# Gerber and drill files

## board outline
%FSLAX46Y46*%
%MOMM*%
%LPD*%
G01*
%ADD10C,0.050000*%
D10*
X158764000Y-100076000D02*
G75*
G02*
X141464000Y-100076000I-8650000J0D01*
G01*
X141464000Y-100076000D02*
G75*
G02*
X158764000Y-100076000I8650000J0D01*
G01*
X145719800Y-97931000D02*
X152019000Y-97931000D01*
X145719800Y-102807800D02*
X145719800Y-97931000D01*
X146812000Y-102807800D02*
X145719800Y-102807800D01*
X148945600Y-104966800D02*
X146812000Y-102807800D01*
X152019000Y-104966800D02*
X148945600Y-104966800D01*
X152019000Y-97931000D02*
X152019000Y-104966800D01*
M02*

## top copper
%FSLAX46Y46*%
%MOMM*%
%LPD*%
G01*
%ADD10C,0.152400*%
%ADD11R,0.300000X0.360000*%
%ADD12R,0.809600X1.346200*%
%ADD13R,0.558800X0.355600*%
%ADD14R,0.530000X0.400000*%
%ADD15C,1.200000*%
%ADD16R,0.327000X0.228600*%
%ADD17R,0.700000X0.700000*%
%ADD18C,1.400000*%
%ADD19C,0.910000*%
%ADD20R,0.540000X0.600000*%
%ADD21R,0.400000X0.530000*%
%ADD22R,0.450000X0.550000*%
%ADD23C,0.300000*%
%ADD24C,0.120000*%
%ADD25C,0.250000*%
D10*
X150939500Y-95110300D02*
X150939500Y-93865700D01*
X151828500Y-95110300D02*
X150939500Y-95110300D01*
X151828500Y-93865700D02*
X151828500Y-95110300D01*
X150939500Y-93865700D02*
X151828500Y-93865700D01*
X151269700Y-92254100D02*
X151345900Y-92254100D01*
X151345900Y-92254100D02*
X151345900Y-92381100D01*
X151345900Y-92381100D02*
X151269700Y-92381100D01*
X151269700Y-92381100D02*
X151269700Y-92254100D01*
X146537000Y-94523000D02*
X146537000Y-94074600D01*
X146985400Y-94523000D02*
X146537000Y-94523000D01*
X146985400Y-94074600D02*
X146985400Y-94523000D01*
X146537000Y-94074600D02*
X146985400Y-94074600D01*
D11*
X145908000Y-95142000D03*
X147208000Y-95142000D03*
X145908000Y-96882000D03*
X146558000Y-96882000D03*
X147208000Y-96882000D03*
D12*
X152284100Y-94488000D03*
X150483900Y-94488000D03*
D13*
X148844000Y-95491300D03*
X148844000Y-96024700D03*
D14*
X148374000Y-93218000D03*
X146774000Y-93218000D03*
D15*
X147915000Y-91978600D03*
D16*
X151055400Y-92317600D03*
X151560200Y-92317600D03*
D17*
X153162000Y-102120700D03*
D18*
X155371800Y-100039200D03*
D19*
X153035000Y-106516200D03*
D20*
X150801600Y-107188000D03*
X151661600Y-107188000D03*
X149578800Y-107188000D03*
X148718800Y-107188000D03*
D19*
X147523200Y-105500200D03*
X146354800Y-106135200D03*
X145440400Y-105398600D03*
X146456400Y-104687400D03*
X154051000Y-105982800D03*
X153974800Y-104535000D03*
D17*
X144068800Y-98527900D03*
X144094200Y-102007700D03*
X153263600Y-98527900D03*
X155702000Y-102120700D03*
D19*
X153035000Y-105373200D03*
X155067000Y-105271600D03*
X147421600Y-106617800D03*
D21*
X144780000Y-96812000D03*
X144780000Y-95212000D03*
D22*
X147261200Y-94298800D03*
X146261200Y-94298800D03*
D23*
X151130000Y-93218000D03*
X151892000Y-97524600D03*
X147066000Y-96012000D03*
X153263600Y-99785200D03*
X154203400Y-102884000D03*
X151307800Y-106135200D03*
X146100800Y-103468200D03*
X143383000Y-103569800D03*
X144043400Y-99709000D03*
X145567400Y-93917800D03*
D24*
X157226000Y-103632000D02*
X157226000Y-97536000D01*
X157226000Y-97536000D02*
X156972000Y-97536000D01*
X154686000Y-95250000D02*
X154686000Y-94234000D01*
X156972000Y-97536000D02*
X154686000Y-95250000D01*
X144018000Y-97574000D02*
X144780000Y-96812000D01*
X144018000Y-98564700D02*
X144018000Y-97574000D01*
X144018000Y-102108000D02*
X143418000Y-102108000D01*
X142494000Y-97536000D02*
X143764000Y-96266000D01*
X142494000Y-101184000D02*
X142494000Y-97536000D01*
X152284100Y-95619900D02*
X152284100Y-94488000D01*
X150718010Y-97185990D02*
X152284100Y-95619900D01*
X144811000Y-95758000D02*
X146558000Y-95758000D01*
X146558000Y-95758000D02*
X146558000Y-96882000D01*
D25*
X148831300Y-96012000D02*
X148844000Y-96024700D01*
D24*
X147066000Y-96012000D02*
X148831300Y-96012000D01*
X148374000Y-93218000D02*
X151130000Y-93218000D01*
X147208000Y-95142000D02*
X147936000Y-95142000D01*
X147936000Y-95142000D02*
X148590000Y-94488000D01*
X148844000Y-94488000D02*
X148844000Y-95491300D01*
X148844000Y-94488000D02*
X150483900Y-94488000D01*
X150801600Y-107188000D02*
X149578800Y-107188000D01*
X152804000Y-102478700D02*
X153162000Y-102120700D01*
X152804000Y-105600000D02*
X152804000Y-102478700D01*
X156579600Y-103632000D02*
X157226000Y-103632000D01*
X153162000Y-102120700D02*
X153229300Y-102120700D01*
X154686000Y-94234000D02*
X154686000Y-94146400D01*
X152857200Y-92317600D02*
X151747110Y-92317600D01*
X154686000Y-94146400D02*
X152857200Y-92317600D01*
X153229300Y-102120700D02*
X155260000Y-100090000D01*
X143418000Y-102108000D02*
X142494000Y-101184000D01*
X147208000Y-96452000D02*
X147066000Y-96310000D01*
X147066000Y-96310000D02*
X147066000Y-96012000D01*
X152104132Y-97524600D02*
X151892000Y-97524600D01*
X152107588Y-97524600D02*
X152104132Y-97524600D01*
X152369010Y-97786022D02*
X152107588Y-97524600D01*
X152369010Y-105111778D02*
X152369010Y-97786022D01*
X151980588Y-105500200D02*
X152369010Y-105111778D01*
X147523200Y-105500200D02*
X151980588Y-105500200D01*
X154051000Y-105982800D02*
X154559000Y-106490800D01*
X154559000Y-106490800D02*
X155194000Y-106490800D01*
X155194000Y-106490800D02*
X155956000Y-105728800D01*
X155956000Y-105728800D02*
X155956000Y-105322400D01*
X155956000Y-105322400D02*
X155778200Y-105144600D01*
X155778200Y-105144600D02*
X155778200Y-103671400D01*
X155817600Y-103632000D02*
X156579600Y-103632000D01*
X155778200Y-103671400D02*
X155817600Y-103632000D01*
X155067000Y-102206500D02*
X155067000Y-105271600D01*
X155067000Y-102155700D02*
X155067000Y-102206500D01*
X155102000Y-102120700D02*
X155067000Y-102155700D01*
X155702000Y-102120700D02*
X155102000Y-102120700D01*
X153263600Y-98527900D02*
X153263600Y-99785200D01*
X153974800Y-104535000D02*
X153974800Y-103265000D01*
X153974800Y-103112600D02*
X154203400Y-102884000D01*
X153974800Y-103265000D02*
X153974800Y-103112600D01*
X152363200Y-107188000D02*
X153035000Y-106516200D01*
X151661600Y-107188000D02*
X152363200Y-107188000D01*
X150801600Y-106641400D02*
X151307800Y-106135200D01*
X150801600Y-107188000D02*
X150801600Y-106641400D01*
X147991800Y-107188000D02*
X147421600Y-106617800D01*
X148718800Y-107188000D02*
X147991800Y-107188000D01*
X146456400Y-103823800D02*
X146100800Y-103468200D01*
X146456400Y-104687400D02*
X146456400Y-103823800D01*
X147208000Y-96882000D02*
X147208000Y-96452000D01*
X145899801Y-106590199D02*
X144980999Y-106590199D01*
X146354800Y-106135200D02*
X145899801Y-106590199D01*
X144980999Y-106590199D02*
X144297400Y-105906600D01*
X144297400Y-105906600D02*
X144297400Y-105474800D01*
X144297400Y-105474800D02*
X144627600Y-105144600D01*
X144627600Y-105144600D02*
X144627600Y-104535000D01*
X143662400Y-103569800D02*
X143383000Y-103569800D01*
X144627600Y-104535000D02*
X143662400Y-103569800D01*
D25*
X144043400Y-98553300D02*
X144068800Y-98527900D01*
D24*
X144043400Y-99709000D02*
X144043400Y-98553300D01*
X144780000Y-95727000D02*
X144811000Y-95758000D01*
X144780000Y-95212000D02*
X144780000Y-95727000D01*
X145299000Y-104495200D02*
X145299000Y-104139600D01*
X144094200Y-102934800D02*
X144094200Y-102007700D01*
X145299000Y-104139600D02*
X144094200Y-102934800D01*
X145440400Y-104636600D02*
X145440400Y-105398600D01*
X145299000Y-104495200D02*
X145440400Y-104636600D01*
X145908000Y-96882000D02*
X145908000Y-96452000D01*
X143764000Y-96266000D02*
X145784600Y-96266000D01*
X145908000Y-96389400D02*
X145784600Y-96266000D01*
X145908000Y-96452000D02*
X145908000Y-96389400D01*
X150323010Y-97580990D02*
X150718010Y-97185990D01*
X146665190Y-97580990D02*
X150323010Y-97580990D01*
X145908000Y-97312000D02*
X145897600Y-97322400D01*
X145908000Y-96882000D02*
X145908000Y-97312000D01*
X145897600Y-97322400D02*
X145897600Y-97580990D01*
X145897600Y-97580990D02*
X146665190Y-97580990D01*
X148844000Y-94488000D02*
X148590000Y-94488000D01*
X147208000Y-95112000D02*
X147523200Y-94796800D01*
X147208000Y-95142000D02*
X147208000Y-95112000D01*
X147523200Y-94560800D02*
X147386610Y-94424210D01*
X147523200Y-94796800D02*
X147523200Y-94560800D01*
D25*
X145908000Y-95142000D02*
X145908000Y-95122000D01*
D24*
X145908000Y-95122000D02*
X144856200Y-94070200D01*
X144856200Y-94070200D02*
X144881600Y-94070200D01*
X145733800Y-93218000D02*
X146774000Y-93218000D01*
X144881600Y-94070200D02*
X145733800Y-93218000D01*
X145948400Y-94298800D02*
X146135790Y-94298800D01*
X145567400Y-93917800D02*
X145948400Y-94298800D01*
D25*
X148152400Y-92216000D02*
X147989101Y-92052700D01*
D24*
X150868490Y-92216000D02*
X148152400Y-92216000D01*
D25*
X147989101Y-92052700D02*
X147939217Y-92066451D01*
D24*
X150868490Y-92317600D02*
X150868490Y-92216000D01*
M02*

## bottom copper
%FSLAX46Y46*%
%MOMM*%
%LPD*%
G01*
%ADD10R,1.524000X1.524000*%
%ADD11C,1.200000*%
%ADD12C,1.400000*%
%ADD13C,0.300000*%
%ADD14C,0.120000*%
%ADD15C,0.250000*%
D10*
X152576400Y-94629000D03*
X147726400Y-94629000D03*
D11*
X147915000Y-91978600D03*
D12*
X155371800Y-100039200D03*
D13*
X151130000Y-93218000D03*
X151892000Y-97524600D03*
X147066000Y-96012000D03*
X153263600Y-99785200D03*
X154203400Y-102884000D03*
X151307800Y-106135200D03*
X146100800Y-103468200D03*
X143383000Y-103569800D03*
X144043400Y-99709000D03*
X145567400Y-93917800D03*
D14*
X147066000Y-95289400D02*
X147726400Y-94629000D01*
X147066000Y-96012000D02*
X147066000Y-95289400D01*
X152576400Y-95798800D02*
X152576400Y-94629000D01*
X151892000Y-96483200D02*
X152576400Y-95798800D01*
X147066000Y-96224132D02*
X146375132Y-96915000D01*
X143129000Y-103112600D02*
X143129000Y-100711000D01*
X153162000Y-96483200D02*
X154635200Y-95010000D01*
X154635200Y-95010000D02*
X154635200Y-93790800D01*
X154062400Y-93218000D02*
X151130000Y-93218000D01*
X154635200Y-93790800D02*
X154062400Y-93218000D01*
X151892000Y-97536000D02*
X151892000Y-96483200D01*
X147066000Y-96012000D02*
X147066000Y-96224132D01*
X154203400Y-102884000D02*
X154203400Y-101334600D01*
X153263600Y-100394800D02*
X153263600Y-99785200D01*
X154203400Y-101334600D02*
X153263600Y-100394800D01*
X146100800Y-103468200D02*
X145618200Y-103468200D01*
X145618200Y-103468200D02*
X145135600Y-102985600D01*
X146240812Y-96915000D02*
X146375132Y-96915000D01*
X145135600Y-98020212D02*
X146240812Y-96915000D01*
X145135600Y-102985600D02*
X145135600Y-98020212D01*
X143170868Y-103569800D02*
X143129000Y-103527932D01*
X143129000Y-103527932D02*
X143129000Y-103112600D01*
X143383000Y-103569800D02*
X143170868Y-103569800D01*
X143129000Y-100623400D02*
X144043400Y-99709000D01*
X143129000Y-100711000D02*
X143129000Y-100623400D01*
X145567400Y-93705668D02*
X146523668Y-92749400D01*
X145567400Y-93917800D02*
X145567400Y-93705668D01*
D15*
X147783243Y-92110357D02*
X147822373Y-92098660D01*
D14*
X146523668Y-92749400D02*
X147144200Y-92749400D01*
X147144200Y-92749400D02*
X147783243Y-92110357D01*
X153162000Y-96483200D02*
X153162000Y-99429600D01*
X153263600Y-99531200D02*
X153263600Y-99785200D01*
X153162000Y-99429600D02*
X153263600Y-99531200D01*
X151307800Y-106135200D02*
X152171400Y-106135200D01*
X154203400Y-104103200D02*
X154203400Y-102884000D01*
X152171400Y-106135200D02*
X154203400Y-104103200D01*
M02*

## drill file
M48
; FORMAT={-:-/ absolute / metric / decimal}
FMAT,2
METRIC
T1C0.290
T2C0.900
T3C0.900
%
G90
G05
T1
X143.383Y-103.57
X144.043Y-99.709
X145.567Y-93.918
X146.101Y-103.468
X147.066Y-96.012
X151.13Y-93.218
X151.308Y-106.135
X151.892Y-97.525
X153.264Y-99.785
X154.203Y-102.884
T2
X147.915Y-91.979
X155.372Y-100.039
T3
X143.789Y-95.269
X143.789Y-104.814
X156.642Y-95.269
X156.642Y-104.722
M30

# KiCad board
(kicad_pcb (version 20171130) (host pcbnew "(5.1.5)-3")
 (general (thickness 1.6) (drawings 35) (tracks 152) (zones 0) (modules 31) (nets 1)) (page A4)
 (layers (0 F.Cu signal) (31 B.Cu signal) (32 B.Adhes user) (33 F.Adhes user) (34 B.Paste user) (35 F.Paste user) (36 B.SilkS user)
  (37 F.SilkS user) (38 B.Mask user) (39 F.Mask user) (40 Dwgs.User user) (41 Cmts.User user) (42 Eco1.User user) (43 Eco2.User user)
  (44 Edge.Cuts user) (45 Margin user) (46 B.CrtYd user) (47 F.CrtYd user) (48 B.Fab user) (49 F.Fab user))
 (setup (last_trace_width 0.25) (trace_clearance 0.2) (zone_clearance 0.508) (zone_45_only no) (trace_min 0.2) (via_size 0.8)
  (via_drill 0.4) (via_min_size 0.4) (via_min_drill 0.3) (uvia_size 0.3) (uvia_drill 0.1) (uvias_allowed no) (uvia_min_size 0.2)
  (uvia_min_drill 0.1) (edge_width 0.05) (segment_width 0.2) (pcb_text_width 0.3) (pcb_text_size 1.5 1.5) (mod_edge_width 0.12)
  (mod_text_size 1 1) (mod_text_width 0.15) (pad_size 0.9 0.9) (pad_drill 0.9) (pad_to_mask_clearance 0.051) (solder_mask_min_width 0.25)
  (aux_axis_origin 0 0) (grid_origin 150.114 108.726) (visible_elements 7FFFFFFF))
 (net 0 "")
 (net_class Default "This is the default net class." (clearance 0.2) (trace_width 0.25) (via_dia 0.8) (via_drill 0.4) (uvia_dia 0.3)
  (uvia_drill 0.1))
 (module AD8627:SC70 (layer F.Cu) (at 146.558 96.012)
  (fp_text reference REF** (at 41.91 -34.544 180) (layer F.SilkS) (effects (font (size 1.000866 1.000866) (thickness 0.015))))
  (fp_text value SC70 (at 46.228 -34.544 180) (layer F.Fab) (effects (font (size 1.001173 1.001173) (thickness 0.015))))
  (pad 5 smd rect (at -0.65 -0.87 180) (size 0.3 0.36) (layers F.Cu F.Paste F.Mask))
  (pad 4 smd rect (at 0.65 -0.87 180) (size 0.3 0.36) (layers F.Cu F.Paste F.Mask))
  (pad 1 smd rect (at -0.65 0.87) (size 0.3 0.36) (layers F.Cu F.Paste F.Mask))
  (pad 2 smd rect (at 0 0.87) (size 0.3 0.36) (layers F.Cu F.Paste F.Mask))
  (pad 3 smd rect (at 0.65 0.87) (size 0.3 0.36) (layers F.Cu F.Paste F.Mask)))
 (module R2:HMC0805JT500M (layer F.Cu) (at 151.384 94.488)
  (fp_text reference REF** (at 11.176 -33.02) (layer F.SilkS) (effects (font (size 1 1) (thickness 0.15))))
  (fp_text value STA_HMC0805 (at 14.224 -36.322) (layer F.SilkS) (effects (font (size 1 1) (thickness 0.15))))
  (fp_line (start -0.4445 0.6223) (end -0.4445 -0.6223) (layer F.Cu) (width 0.1524))
  (fp_line (start 0.4445 0.6223) (end -0.4445 0.6223) (layer F.Cu) (width 0.1524))
  (fp_line (start 0.4445 -0.6223) (end 0.4445 0.6223) (layer F.Cu) (width 0.1524))
  (fp_line (start -0.4445 -0.6223) (end 0.4445 -0.6223) (layer F.Cu) (width 0.1524))
  (pad 2 smd rect (at 0.9001 0) (size 0.8096 1.3462) (layers F.Cu F.Paste F.Mask))
  (pad 1 smd rect (at -0.9001 0) (size 0.8096 1.3462) (layers F.Cu F.Paste F.Mask)))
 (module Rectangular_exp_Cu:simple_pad (layer F.Cu) (at 150.2664 94.629)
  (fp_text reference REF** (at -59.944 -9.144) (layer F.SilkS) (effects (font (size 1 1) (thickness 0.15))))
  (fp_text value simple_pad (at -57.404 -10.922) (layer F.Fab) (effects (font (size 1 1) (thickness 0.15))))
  (pad 2 smd rect (at 2.31 0) (size 1.524 1.524) (layers B.Cu))
  (pad 1 smd rect (at -2.54 0) (size 1.524 1.524) (layers B.Cu)))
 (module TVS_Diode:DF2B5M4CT (layer F.Cu) (at 148.844 95.758 90)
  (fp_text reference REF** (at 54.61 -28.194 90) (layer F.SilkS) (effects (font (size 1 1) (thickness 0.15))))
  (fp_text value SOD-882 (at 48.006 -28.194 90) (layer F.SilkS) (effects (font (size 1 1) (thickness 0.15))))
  (pad 2 smd rect (at 0.2667 0 90) (size 0.3556 0.5588) (layers F.Cu F.Paste F.Mask))
  (pad 1 smd rect (at -0.2667 0 90) (size 0.3556 0.5588) (layers F.Cu F.Paste F.Mask)))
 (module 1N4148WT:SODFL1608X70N (layer F.Cu) (at 147.574 93.218)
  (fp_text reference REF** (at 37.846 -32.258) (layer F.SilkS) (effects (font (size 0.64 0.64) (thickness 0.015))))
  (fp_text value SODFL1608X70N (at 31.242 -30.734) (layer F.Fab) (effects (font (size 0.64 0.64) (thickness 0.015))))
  (pad A smd rect (at 0.8 0) (size 0.53 0.4) (layers F.Cu F.Paste F.Mask))
  (pad C smd rect (at -0.8 0) (size 0.53 0.4) (layers F.Cu F.Paste F.Mask)))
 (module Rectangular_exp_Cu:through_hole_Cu (layer F.Cu) (at 148.209 92.47)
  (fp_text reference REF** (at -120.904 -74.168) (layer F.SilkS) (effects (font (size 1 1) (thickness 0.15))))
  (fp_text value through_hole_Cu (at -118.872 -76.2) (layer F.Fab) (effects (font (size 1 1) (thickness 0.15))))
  (pad 1 thru_hole circle (at -0.294 -0.4914) (size 1.2 1.2) (drill 0.9) (layers *.Mask F.Cu)))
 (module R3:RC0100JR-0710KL (layer F.Cu) (at 151.3078 92.3176)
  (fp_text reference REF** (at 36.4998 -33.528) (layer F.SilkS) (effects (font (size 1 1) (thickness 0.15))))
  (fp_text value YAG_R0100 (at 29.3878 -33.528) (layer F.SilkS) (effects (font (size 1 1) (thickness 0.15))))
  (fp_line (start -0.0381 -0.0635) (end 0.0381 -0.0635) (layer F.Cu) (width 0.1524))
  (fp_line (start 0.0381 -0.0635) (end 0.0381 0.0635) (layer F.Cu) (width 0.1524))
  (fp_line (start 0.0381 0.0635) (end -0.0381 0.0635) (layer F.Cu) (width 0.1524))
  (fp_line (start -0.0381 0.0635) (end -0.0381 -0.0635) (layer F.Cu) (width 0.1524))
  (pad 1 smd rect (at -0.2524 0) (size 0.327 0.2286) (layers F.Cu F.Paste F.Mask))
  (pad 2 smd rect (at 0.2524 0) (size 0.327 0.2286) (layers F.Cu F.Paste F.Mask)))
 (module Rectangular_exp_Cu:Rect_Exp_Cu (layer F.Cu) (at 153.162 102.108)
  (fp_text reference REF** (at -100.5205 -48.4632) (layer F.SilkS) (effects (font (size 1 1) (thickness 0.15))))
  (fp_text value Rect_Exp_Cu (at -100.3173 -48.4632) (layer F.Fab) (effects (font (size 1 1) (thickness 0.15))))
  (pad 1 smd rect (at 0 0.0127) (size 0.7 0.7) (layers F.Cu F.Paste F.Mask)))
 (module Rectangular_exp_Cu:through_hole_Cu (layer F.Cu) (at 156.0678 99.0092)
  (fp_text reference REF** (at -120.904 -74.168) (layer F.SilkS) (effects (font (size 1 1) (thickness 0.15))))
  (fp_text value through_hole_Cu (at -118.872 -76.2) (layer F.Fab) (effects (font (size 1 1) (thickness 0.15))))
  (pad 1 thru_hole circle (at -0.696 1.03) (size 1.4 1.4) (drill 0.9) (layers *.Mask F.Cu)))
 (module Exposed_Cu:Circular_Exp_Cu (layer F.Cu) (at 152.885 106.7302)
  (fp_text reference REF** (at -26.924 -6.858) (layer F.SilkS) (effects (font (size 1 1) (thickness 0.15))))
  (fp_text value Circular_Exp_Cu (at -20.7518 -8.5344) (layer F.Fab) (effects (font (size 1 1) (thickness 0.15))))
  (pad 1 smd circle (at 0.15 -0.214) (size 0.91 0.91) (layers F.Cu F.Paste F.Mask)))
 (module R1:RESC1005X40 (layer F.Cu) (at 151.2316 107.188)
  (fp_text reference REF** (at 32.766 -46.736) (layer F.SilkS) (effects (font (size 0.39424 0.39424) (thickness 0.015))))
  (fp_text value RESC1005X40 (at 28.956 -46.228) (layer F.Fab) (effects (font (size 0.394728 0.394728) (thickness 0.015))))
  (pad 1 smd rect (at -0.43 0) (size 0.54 0.6) (layers F.Cu F.Paste F.Mask))
  (pad 2 smd rect (at 0.43 0) (size 0.54 0.6) (layers F.Cu F.Paste F.Mask)))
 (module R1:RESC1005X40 (layer F.Cu) (at 149.1488 107.188)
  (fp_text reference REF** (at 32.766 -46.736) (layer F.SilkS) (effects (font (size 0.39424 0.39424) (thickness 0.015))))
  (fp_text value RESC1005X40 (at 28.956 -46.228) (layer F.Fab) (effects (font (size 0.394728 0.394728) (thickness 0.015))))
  (pad 2 smd rect (at 0.43 0) (size 0.54 0.6) (layers F.Cu F.Paste F.Mask))
  (pad 1 smd rect (at -0.43 0) (size 0.54 0.6) (layers F.Cu F.Paste F.Mask)))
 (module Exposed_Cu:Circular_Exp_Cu (layer F.Cu) (at 147.8032 105.8182)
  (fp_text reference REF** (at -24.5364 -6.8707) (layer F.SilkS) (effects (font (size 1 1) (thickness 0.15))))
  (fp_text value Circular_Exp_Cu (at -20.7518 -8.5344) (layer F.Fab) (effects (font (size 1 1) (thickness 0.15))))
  (pad 1 smd circle (at -0.28 -0.318) (size 0.91 0.91) (layers F.Cu F.Paste F.Mask)))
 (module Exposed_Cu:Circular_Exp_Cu (layer F.Cu) (at 146.7268 106.3562)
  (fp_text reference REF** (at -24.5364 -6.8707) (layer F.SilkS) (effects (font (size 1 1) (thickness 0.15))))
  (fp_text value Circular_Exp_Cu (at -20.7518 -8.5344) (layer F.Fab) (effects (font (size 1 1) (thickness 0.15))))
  (pad 1 smd circle (at -0.372 -0.221) (size 0.91 0.91) (layers F.Cu F.Paste F.Mask)))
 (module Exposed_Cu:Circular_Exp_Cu (layer F.Cu) (at 145.3786 105.5118)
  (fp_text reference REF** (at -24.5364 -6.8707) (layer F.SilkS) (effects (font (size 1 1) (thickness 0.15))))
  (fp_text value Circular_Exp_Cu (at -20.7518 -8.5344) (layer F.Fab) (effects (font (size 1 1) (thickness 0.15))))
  (pad 1 smd circle (at 0.0618 -0.1132) (size 0.91 0.91) (layers F.Cu F.Paste F.Mask)))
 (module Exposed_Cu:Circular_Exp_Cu (layer F.Cu) (at 146.7554 105.2854)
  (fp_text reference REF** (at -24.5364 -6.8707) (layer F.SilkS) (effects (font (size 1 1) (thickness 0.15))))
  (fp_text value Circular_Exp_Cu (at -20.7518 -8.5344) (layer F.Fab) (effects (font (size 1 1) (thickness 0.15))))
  (pad 1 smd circle (at -0.299 -0.598) (size 0.91 0.91) (layers F.Cu F.Paste F.Mask)))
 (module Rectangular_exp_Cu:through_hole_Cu (layer F.Cu) (at 160.8582 95.518)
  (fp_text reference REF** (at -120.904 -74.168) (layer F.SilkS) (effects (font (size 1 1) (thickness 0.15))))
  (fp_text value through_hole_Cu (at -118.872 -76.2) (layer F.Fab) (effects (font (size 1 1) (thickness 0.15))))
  (pad "" np_thru_hole circle (at -4.2158 -0.249) (size 0.9 0.9) (drill 0.9) (layers *.Cu *.Mask)))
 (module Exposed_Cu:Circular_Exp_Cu (layer F.Cu) (at 153.645 106.4578)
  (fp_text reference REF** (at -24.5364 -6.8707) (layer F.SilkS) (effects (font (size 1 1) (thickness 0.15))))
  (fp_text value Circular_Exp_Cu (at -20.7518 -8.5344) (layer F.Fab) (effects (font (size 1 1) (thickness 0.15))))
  (pad 1 smd circle (at 0.406 -0.475) (size 0.91 0.91) (layers F.Cu F.Paste F.Mask)))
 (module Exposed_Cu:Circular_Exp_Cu (layer F.Cu) (at 153.9228 105.133)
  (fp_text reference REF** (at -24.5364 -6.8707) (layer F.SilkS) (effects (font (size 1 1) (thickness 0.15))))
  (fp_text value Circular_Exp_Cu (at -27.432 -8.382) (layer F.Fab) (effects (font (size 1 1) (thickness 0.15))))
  (pad 1 smd circle (at 0.052 -0.598) (size 0.91 0.91) (layers F.Cu F.Paste F.Mask)))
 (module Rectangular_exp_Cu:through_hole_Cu (layer F.Cu) (at 159.4358 103.3412)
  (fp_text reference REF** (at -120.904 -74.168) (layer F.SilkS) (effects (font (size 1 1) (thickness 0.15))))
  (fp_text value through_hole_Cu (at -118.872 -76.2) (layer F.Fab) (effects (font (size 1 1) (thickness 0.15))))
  (pad "" np_thru_hole circle (at -2.7934 1.3806) (size 0.9 0.9) (drill 0.9) (layers *.Cu *.Mask)))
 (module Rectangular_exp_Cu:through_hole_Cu (layer F.Cu) (at 138.6332 103.6484)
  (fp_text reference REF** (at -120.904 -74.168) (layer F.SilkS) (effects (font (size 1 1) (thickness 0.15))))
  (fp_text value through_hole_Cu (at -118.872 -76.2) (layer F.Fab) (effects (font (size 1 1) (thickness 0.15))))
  (pad "" np_thru_hole circle (at 5.1562 1.166) (size 0.9 0.9) (drill 0.9) (layers *.Cu *.Mask)))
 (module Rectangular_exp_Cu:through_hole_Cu (layer F.Cu) (at 141.5832 93.4162)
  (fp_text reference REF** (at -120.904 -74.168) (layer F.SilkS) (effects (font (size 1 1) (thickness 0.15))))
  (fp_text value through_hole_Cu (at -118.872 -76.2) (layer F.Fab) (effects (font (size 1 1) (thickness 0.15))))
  (pad "" np_thru_hole circle (at 2.2062 1.8528) (size 0.9 0.9) (drill 0.9) (layers *.Cu *.Mask)))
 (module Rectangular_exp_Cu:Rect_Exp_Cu (layer F.Cu) (at 144.0688 98.5152)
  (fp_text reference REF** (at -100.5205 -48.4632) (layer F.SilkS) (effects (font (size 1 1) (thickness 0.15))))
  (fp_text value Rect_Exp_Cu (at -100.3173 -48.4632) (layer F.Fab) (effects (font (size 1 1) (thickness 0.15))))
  (pad 1 smd rect (at 0 0.0127) (size 0.7 0.7) (layers F.Cu F.Paste F.Mask)))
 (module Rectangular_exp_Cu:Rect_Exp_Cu (layer F.Cu) (at 144.0942 101.995)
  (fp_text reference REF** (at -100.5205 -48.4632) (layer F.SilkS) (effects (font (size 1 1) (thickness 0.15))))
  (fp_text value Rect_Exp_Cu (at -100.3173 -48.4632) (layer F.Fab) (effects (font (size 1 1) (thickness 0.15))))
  (pad 1 smd rect (at 0 0.0127) (size 0.7 0.7) (layers F.Cu F.Paste F.Mask)))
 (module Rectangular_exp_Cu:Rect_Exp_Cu (layer F.Cu) (at 153.2636 98.5152)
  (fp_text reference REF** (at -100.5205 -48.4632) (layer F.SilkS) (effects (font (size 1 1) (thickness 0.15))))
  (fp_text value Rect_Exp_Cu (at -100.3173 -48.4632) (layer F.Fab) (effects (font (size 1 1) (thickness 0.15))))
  (pad 1 smd rect (at 0 0.0127) (size 0.7 0.7) (layers F.Cu F.Paste F.Mask)))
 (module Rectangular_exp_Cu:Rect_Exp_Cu (layer F.Cu) (at 155.702 102.108)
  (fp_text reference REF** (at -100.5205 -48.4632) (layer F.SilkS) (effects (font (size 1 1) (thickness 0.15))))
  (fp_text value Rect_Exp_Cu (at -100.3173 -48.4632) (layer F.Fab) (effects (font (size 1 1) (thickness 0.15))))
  (pad 1 smd rect (at 0 0.0127) (size 0.7 0.7) (layers F.Cu F.Paste F.Mask)))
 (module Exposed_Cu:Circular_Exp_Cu (layer F.Cu) (at 153.1263 105.6912)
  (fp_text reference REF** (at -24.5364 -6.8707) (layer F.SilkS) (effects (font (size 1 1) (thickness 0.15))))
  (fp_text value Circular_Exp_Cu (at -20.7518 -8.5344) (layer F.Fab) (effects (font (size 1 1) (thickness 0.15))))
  (pad 1 smd circle (at -0.0913 -0.318) (size 0.91 0.91) (layers F.Cu F.Paste F.Mask)))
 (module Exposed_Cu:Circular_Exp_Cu (layer F.Cu) (at 154.431 105.9296)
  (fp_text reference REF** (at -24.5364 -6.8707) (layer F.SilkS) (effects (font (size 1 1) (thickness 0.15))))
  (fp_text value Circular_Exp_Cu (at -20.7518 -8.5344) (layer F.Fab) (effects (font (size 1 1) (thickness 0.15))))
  (pad 1 smd circle (at 0.636 -0.658) (size 0.91 0.91) (layers F.Cu F.Paste F.Mask)))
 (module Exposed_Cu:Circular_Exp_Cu (layer F.Cu) (at 147.7676 106.8318)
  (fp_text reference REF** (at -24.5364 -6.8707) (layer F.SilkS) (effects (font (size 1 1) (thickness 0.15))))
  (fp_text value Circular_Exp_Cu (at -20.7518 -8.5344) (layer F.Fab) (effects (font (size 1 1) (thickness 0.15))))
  (pad 1 smd circle (at -0.346 -0.214) (size 0.91 0.91) (layers F.Cu F.Paste F.Mask)))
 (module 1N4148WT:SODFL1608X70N (layer F.Cu) (at 144.78 96.012 90)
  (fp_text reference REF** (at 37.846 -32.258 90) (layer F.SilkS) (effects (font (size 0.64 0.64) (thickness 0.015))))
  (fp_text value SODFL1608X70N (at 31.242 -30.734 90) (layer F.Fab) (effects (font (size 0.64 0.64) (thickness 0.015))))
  (pad C smd rect (at -0.8 0 90) (size 0.53 0.4) (layers F.Cu F.Paste F.Mask))
  (pad A smd rect (at 0.8 0 90) (size 0.53 0.4) (layers F.Cu F.Paste F.Mask)))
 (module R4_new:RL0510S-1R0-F (layer F.Cu) (at 146.7612 94.2988)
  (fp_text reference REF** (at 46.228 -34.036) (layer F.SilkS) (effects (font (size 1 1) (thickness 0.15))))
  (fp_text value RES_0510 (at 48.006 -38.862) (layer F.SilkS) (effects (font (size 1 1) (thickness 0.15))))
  (fp_line (start -0.2242 0.2242) (end -0.2242 -0.2242) (layer F.Cu) (width 0.1524))
  (fp_line (start 0.2242 0.2242) (end -0.2242 0.2242) (layer F.Cu) (width 0.1524))
  (fp_line (start 0.2242 -0.2242) (end 0.2242 0.2242) (layer F.Cu) (width 0.1524))
  (fp_line (start -0.2242 -0.2242) (end 0.2242 -0.2242) (layer F.Cu) (width 0.1524))
  (pad 2 smd rect (at 0.5 0) (size 0.45 0.55) (layers F.Cu F.Paste F.Mask))
  (pad 1 smd rect (at -0.5 0) (size 0.45 0.55) (layers F.Cu F.Paste F.Mask)))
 (gr_circle (center 150.114 100.076) (end 158.764 100.076) (layer Edge.Cuts) (width 0.05))
 (gr_line (start 145.7198 97.931) (end 152.019 97.931) (layer Edge.Cuts) (width 0.05))
 (gr_line (start 145.7198 102.8078) (end 145.7198 97.931) (layer Edge.Cuts) (width 0.05))
 (gr_line (start 146.812 102.8078) (end 145.7198 102.8078) (layer Edge.Cuts) (width 0.05))
 (gr_line (start 148.9456 104.9668) (end 146.812 102.8078) (layer Edge.Cuts) (width 0.05))
 (gr_line (start 152.019 104.9668) (end 148.9456 104.9668) (layer Edge.Cuts) (width 0.05))
 (gr_line (start 152.019 97.931) (end 152.019 104.9668) (layer Edge.Cuts) (width 0.05))
 (via (at 151.13 93.218) (size 0.3) (drill 0.29) (layers F.Cu B.Cu) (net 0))
 (via (at 151.892 97.5246) (size 0.3) (drill 0.29) (layers F.Cu B.Cu) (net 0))
 (segment (start 157.226 103.632) (end 157.226 97.536) (width 0.12) (layer F.Cu) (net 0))
 (segment (start 157.226 97.536) (end 156.972 97.536) (width 0.12) (layer F.Cu) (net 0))
 (segment (start 154.686 95.25) (end 154.686 94.234) (width 0.12) (layer F.Cu) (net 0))
 (segment (start 156.972 97.536) (end 154.686 95.25) (width 0.12) (layer F.Cu) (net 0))
 (segment (start 144.018 97.574) (end 144.78 96.812) (width 0.12) (layer F.Cu) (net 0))
 (segment (start 144.018 98.5647) (end 144.018 97.574) (width 0.12) (layer F.Cu) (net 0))
 (segment (start 144.018 102.108) (end 143.418 102.108) (width 0.12) (layer F.Cu) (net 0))
 (segment (start 142.494 97.536) (end 143.764 96.266) (width 0.12) (layer F.Cu) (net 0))
 (segment (start 142.494 101.184) (end 142.494 97.536) (width 0.12) (layer F.Cu) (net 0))
 (segment (start 152.2841 95.6199) (end 152.2841 94.488) (width 0.12) (layer F.Cu) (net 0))
 (segment (start 150.71801 97.18599) (end 152.2841 95.6199) (width 0.12) (layer F.Cu) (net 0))
 (segment (start 144.811 95.758) (end 146.558 95.758) (width 0.12) (layer F.Cu) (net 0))
 (segment (start 146.558 95.758) (end 146.558 96.882) (width 0.12) (layer F.Cu) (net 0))
 (segment (start 148.8313 96.012) (end 148.844 96.0247) (width 0.25) (layer F.Cu) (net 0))
 (segment (start 147.066 96.012) (end 148.8313 96.012) (width 0.12) (layer F.Cu) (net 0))
 (segment (start 148.374 93.218) (end 151.13 93.218) (width 0.12) (layer F.Cu) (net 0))
 (segment (start 147.208 95.142) (end 147.936 95.142) (width 0.12) (layer F.Cu) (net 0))
 (segment (start 147.936 95.142) (end 148.59 94.488) (width 0.12) (layer F.Cu) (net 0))
 (segment (start 148.844 94.488) (end 148.844 95.4913) (width 0.12) (layer F.Cu) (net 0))
 (segment (start 148.844 94.488) (end 150.4839 94.488) (width 0.12) (layer F.Cu) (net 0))
 (segment (start 150.8016 107.188) (end 149.5788 107.188) (width 0.12) (layer F.Cu) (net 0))
 (segment (start 152.804 102.4787) (end 153.162 102.1207) (width 0.12) (layer F.Cu) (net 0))
 (segment (start 152.804 105.6) (end 152.804 102.4787) (width 0.12) (layer F.Cu) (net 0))
 (segment (start 156.5796 103.632) (end 157.226 103.632) (width 0.12) (layer F.Cu) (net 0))
 (segment (start 153.162 102.1207) (end 153.2293 102.1207) (width 0.12) (layer F.Cu) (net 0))
 (segment (start 154.686 94.234) (end 154.686 94.1464) (width 0.12) (layer F.Cu) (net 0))
 (segment (start 152.8572 92.3176) (end 151.74711 92.3176) (width 0.12) (layer F.Cu) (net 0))
 (segment (start 154.686 94.1464) (end 152.8572 92.3176) (width 0.12) (layer F.Cu) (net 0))
 (segment (start 147.066 95.2894) (end 147.7264 94.629) (width 0.12) (layer B.Cu) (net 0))
 (segment (start 147.066 96.012) (end 147.066 95.2894) (width 0.12) (layer B.Cu) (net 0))
 (segment (start 152.5764 95.7988) (end 152.5764 94.629) (width 0.12) (layer B.Cu) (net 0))
 (segment (start 151.892 96.4832) (end 152.5764 95.7988) (width 0.12) (layer B.Cu) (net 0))
 (segment (start 147.066 96.224132) (end 146.375132 96.915) (width 0.12) (layer B.Cu) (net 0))
 (segment (start 143.129 103.1126) (end 143.129 100.711) (width 0.12) (layer B.Cu) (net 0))
 (segment (start 153.162 96.4832) (end 154.6352 95.01) (width 0.12) (layer B.Cu) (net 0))
 (segment (start 154.6352 95.01) (end 154.6352 93.7908) (width 0.12) (layer B.Cu) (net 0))
 (segment (start 154.0624 93.218) (end 151.13 93.218) (width 0.12) (layer B.Cu) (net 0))
 (segment (start 154.6352 93.7908) (end 154.0624 93.218) (width 0.12) (layer B.Cu) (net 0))
 (segment (start 151.892 97.536) (end 151.892 96.4832) (width 0.12) (layer B.Cu) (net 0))
 (segment (start 153.2293 102.1207) (end 155.26 100.09) (width 0.12) (layer F.Cu) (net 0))
 (segment (start 143.418 102.108) (end 142.494 101.184) (width 0.12) (layer F.Cu) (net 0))
 (segment (start 147.066 96.012) (end 147.066 96.224132) (width 0.12) (layer B.Cu) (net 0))
 (segment (start 147.208 96.452) (end 147.066 96.31) (width 0.12) (layer F.Cu) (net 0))
 (segment (start 147.066 96.31) (end 147.066 96.012) (width 0.12) (layer F.Cu) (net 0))
 (via (at 147.066 96.012) (size 0.3) (drill 0.29) (layers F.Cu B.Cu) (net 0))
 (segment (start 152.104132 97.5246) (end 151.892 97.5246) (width 0.12) (layer F.Cu) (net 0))
 (segment (start 152.107588 97.5246) (end 152.104132 97.5246) (width 0.12) (layer F.Cu) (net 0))
 (segment (start 152.36901 97.786022) (end 152.107588 97.5246) (width 0.12) (layer F.Cu) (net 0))
 (segment (start 152.36901 105.111778) (end 152.36901 97.786022) (width 0.12) (layer F.Cu) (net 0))
 (segment (start 151.980588 105.5002) (end 152.36901 105.111778) (width 0.12) (layer F.Cu) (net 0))
 (segment (start 147.5232 105.5002) (end 151.980588 105.5002) (width 0.12) (layer F.Cu) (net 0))
 (segment (start 154.051 105.9828) (end 154.559 106.4908) (width 0.12) (layer F.Cu) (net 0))
 (segment (start 154.559 106.4908) (end 155.194 106.4908) (width 0.12) (layer F.Cu) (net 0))
 (segment (start 155.194 106.4908) (end 155.956 105.7288) (width 0.12) (layer F.Cu) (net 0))
 (segment (start 155.956 105.7288) (end 155.956 105.3224) (width 0.12) (layer F.Cu) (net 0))
 (segment (start 155.956 105.3224) (end 155.7782 105.1446) (width 0.12) (layer F.Cu) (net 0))
 (segment (start 155.7782 105.1446) (end 155.7782 103.6714) (width 0.12) (layer F.Cu) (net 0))
 (segment (start 155.8176 103.632) (end 156.5796 103.632) (width 0.12) (layer F.Cu) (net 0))
 (segment (start 155.7782 103.6714) (end 155.8176 103.632) (width 0.12) (layer F.Cu) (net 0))
 (segment (start 155.067 102.2065) (end 155.067 105.2716) (width 0.12) (layer F.Cu) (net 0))
 (segment (start 155.067 102.1557) (end 155.067 102.2065) (width 0.12) (layer F.Cu) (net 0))
 (segment (start 155.102 102.1207) (end 155.067 102.1557) (width 0.12) (layer F.Cu) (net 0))
 (segment (start 155.702 102.1207) (end 155.102 102.1207) (width 0.12) (layer F.Cu) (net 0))
 (via (at 153.2636 99.7852) (size 0.3) (drill 0.29) (layers F.Cu B.Cu) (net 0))
 (segment (start 153.2636 98.5279) (end 153.2636 99.7852) (width 0.12) (layer F.Cu) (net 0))
 (via (at 154.2034 102.884) (size 0.3) (drill 0.29) (layers F.Cu B.Cu) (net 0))
 (segment (start 153.9748 104.535) (end 153.9748 103.265) (width 0.12) (layer F.Cu) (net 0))
 (segment (start 153.9748 103.1126) (end 154.2034 102.884) (width 0.12) (layer F.Cu) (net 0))
 (segment (start 153.9748 103.265) (end 153.9748 103.1126) (width 0.12) (layer F.Cu) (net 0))
 (segment (start 154.2034 102.884) (end 154.2034 101.3346) (width 0.12) (layer B.Cu) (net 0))
 (segment (start 153.2636 100.3948) (end 153.2636 99.7852) (width 0.12) (layer B.Cu) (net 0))
 (segment (start 154.2034 101.3346) (end 153.2636 100.3948) (width 0.12) (layer B.Cu) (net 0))
 (segment (start 152.3632 107.188) (end 153.035 106.5162) (width 0.12) (layer F.Cu) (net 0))
 (segment (start 151.6616 107.188) (end 152.3632 107.188) (width 0.12) (layer F.Cu) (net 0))
 (via (at 151.3078 106.1352) (size 0.3) (drill 0.29) (layers F.Cu B.Cu) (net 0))
 (segment (start 150.8016 106.6414) (end 151.3078 106.1352) (width 0.12) (layer F.Cu) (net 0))
 (segment (start 150.8016 107.188) (end 150.8016 106.6414) (width 0.12) (layer F.Cu) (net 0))
 (segment (start 147.9918 107.188) (end 147.4216 106.6178) (width 0.12) (layer F.Cu) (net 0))
 (segment (start 148.7188 107.188) (end 147.9918 107.188) (width 0.12) (layer F.Cu) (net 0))
 (via (at 146.1008 103.4682) (size 0.3) (drill 0.29) (layers F.Cu B.Cu) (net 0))
 (segment (start 146.4564 103.8238) (end 146.1008 103.4682) (width 0.12) (layer F.Cu) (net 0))
 (segment (start 146.4564 104.6874) (end 146.4564 103.8238) (width 0.12) (layer F.Cu) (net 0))
 (segment (start 146.1008 103.4682) (end 145.6182 103.4682) (width 0.12) (layer B.Cu) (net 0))
 (segment (start 145.6182 103.4682) (end 145.1356 102.9856) (width 0.12) (layer B.Cu) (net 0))
 (segment (start 146.240812 96.915) (end 146.375132 96.915) (width 0.12) (layer B.Cu) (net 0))
 (segment (start 145.1356 98.020212) (end 146.240812 96.915) (width 0.12) (layer B.Cu) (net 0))
 (segment (start 145.1356 102.9856) (end 145.1356 98.020212) (width 0.12) (layer B.Cu) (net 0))
 (segment (start 147.208 96.882) (end 147.208 96.452) (width 0.12) (layer F.Cu) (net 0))
 (via (at 143.383 103.5698) (size 0.3) (drill 0.29) (layers F.Cu B.Cu) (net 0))
 (segment (start 145.899801 106.590199) (end 144.980999 106.590199) (width 0.12) (layer F.Cu) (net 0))
 (segment (start 146.3548 106.1352) (end 145.899801 106.590199) (width 0.12) (layer F.Cu) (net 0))
 (segment (start 144.980999 106.590199) (end 144.2974 105.9066) (width 0.12) (layer F.Cu) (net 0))
 (segment (start 144.2974 105.9066) (end 144.2974 105.4748) (width 0.12) (layer F.Cu) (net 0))
 (segment (start 144.2974 105.4748) (end 144.6276 105.1446) (width 0.12) (layer F.Cu) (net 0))
 (segment (start 144.6276 105.1446) (end 144.6276 104.535) (width 0.12) (layer F.Cu) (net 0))
 (segment (start 143.6624 103.5698) (end 143.383 103.5698) (width 0.12) (layer F.Cu) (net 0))
 (segment (start 144.6276 104.535) (end 143.6624 103.5698) (width 0.12) (layer F.Cu) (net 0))
 (via (at 144.0434 99.709) (size 0.3) (drill 0.29) (layers F.Cu B.Cu) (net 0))
 (segment (start 143.170868 103.5698) (end 143.129 103.527932) (width 0.12) (layer B.Cu) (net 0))
 (segment (start 143.129 103.527932) (end 143.129 103.1126) (width 0.12) (layer B.Cu) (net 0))
 (segment (start 143.383 103.5698) (end 143.170868 103.5698) (width 0.12) (layer B.Cu) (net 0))
 (segment (start 143.129 100.6234) (end 144.0434 99.709) (width 0.12) (layer B.Cu) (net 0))
 (segment (start 143.129 100.711) (end 143.129 100.6234) (width 0.12) (layer B.Cu) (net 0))
 (segment (start 144.0434 98.5533) (end 144.0688 98.5279) (width 0.25) (layer F.Cu) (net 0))
 (segment (start 144.0434 99.709) (end 144.0434 98.5533) (width 0.12) (layer F.Cu) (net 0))
 (segment (start 144.78 95.727) (end 144.811 95.758) (width 0.12) (layer F.Cu) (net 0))
 (segment (start 144.78 95.212) (end 144.78 95.727) (width 0.12) (layer F.Cu) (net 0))
 (segment (start 145.299 104.4952) (end 145.299 104.1396) (width 0.12) (layer F.Cu) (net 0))
 (segment (start 144.0942 102.9348) (end 144.0942 102.0077) (width 0.12) (layer F.Cu) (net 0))
 (segment (start 145.299 104.1396) (end 144.0942 102.9348) (width 0.12) (layer F.Cu) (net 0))
 (segment (start 145.4404 104.6366) (end 145.4404 105.3986) (width 0.12) (layer F.Cu) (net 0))
 (segment (start 145.299 104.4952) (end 145.4404 104.6366) (width 0.12) (layer F.Cu) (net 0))
 (segment (start 145.908 96.882) (end 145.908 96.452) (width 0.12) (layer F.Cu) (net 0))
 (segment (start 143.764 96.266) (end 145.7846 96.266) (width 0.12) (layer F.Cu) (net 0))
 (segment (start 145.908 96.3894) (end 145.7846 96.266) (width 0.12) (layer F.Cu) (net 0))
 (segment (start 145.908 96.452) (end 145.908 96.3894) (width 0.12) (layer F.Cu) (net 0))
 (segment (start 150.32301 97.58099) (end 150.71801 97.18599) (width 0.12) (layer F.Cu) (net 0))
 (segment (start 146.66519 97.58099) (end 150.32301 97.58099) (width 0.12) (layer F.Cu) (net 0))
 (segment (start 145.908 97.312) (end 145.8976 97.3224) (width 0.12) (layer F.Cu) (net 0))
 (segment (start 145.908 96.882) (end 145.908 97.312) (width 0.12) (layer F.Cu) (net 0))
 (segment (start 145.8976 97.3224) (end 145.8976 97.58099) (width 0.12) (layer F.Cu) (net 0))
 (segment (start 145.8976 97.58099) (end 146.66519 97.58099) (width 0.12) (layer F.Cu) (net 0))
 (segment (start 148.844 94.488) (end 148.59 94.488) (width 0.12) (layer F.Cu) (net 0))
 (segment (start 147.208 95.112) (end 147.5232 94.7968) (width 0.12) (layer F.Cu) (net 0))
 (segment (start 147.208 95.142) (end 147.208 95.112) (width 0.12) (layer F.Cu) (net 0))
 (segment (start 147.5232 94.5608) (end 147.38661 94.42421) (width 0.12) (layer F.Cu) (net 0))
 (segment (start 147.5232 94.7968) (end 147.5232 94.5608) (width 0.12) (layer F.Cu) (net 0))
 (segment (start 145.908 95.142) (end 145.908 95.122) (width 0.25) (layer F.Cu) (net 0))
 (segment (start 145.908 95.122) (end 144.8562 94.0702) (width 0.12) (layer F.Cu) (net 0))
 (segment (start 144.8562 94.0702) (end 144.8816 94.0702) (width 0.12) (layer F.Cu) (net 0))
 (segment (start 145.7338 93.218) (end 146.774 93.218) (width 0.12) (layer F.Cu) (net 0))
 (segment (start 144.8816 94.0702) (end 145.7338 93.218) (width 0.12) (layer F.Cu) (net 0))
 (via (at 145.5674 93.9178) (size 0.3) (drill 0.29) (layers F.Cu B.Cu) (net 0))
 (segment (start 145.9484 94.2988) (end 146.13579 94.2988) (width 0.12) (layer F.Cu) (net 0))
 (segment (start 145.5674 93.9178) (end 145.9484 94.2988) (width 0.12) (layer F.Cu) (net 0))
 (segment (start 145.5674 93.705668) (end 146.523668 92.7494) (width 0.12) (layer B.Cu) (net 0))
 (segment (start 145.5674 93.9178) (end 145.5674 93.705668) (width 0.12) (layer B.Cu) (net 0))
 (segment (start 147.783243 92.110357) (end 147.822373 92.09866) (width 0.25) (layer B.Cu) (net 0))
 (segment (start 146.523668 92.7494) (end 147.1442 92.7494) (width 0.12) (layer B.Cu) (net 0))
 (segment (start 147.1442 92.7494) (end 147.783243 92.110357) (width 0.12) (layer B.Cu) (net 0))
 (segment (start 148.1524 92.216) (end 147.989101 92.0527) (width 0.25) (layer F.Cu) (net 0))
 (segment (start 150.86849 92.216) (end 148.1524 92.216) (width 0.12) (layer F.Cu) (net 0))
 (segment (start 147.989101 92.0527) (end 147.939217 92.066451) (width 0.25) (layer F.Cu) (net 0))
 (segment (start 150.86849 92.3176) (end 150.86849 92.216) (width 0.12) (layer F.Cu) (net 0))
 (segment (start 153.162 96.4832) (end 153.162 99.4296) (width 0.12) (layer B.Cu) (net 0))
 (segment (start 153.2636 99.5312) (end 153.2636 99.7852) (width 0.12) (layer B.Cu) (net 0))
 (segment (start 153.162 99.4296) (end 153.2636 99.5312) (width 0.12) (layer B.Cu) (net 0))
 (segment (start 151.3078 106.1352) (end 152.1714 106.1352) (width 0.12) (layer B.Cu) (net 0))
 (segment (start 154.2034 104.1032) (end 154.2034 102.884) (width 0.12) (layer B.Cu) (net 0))
 (segment (start 152.1714 106.1352) (end 154.2034 104.1032) (width 0.12) (layer B.Cu) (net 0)))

